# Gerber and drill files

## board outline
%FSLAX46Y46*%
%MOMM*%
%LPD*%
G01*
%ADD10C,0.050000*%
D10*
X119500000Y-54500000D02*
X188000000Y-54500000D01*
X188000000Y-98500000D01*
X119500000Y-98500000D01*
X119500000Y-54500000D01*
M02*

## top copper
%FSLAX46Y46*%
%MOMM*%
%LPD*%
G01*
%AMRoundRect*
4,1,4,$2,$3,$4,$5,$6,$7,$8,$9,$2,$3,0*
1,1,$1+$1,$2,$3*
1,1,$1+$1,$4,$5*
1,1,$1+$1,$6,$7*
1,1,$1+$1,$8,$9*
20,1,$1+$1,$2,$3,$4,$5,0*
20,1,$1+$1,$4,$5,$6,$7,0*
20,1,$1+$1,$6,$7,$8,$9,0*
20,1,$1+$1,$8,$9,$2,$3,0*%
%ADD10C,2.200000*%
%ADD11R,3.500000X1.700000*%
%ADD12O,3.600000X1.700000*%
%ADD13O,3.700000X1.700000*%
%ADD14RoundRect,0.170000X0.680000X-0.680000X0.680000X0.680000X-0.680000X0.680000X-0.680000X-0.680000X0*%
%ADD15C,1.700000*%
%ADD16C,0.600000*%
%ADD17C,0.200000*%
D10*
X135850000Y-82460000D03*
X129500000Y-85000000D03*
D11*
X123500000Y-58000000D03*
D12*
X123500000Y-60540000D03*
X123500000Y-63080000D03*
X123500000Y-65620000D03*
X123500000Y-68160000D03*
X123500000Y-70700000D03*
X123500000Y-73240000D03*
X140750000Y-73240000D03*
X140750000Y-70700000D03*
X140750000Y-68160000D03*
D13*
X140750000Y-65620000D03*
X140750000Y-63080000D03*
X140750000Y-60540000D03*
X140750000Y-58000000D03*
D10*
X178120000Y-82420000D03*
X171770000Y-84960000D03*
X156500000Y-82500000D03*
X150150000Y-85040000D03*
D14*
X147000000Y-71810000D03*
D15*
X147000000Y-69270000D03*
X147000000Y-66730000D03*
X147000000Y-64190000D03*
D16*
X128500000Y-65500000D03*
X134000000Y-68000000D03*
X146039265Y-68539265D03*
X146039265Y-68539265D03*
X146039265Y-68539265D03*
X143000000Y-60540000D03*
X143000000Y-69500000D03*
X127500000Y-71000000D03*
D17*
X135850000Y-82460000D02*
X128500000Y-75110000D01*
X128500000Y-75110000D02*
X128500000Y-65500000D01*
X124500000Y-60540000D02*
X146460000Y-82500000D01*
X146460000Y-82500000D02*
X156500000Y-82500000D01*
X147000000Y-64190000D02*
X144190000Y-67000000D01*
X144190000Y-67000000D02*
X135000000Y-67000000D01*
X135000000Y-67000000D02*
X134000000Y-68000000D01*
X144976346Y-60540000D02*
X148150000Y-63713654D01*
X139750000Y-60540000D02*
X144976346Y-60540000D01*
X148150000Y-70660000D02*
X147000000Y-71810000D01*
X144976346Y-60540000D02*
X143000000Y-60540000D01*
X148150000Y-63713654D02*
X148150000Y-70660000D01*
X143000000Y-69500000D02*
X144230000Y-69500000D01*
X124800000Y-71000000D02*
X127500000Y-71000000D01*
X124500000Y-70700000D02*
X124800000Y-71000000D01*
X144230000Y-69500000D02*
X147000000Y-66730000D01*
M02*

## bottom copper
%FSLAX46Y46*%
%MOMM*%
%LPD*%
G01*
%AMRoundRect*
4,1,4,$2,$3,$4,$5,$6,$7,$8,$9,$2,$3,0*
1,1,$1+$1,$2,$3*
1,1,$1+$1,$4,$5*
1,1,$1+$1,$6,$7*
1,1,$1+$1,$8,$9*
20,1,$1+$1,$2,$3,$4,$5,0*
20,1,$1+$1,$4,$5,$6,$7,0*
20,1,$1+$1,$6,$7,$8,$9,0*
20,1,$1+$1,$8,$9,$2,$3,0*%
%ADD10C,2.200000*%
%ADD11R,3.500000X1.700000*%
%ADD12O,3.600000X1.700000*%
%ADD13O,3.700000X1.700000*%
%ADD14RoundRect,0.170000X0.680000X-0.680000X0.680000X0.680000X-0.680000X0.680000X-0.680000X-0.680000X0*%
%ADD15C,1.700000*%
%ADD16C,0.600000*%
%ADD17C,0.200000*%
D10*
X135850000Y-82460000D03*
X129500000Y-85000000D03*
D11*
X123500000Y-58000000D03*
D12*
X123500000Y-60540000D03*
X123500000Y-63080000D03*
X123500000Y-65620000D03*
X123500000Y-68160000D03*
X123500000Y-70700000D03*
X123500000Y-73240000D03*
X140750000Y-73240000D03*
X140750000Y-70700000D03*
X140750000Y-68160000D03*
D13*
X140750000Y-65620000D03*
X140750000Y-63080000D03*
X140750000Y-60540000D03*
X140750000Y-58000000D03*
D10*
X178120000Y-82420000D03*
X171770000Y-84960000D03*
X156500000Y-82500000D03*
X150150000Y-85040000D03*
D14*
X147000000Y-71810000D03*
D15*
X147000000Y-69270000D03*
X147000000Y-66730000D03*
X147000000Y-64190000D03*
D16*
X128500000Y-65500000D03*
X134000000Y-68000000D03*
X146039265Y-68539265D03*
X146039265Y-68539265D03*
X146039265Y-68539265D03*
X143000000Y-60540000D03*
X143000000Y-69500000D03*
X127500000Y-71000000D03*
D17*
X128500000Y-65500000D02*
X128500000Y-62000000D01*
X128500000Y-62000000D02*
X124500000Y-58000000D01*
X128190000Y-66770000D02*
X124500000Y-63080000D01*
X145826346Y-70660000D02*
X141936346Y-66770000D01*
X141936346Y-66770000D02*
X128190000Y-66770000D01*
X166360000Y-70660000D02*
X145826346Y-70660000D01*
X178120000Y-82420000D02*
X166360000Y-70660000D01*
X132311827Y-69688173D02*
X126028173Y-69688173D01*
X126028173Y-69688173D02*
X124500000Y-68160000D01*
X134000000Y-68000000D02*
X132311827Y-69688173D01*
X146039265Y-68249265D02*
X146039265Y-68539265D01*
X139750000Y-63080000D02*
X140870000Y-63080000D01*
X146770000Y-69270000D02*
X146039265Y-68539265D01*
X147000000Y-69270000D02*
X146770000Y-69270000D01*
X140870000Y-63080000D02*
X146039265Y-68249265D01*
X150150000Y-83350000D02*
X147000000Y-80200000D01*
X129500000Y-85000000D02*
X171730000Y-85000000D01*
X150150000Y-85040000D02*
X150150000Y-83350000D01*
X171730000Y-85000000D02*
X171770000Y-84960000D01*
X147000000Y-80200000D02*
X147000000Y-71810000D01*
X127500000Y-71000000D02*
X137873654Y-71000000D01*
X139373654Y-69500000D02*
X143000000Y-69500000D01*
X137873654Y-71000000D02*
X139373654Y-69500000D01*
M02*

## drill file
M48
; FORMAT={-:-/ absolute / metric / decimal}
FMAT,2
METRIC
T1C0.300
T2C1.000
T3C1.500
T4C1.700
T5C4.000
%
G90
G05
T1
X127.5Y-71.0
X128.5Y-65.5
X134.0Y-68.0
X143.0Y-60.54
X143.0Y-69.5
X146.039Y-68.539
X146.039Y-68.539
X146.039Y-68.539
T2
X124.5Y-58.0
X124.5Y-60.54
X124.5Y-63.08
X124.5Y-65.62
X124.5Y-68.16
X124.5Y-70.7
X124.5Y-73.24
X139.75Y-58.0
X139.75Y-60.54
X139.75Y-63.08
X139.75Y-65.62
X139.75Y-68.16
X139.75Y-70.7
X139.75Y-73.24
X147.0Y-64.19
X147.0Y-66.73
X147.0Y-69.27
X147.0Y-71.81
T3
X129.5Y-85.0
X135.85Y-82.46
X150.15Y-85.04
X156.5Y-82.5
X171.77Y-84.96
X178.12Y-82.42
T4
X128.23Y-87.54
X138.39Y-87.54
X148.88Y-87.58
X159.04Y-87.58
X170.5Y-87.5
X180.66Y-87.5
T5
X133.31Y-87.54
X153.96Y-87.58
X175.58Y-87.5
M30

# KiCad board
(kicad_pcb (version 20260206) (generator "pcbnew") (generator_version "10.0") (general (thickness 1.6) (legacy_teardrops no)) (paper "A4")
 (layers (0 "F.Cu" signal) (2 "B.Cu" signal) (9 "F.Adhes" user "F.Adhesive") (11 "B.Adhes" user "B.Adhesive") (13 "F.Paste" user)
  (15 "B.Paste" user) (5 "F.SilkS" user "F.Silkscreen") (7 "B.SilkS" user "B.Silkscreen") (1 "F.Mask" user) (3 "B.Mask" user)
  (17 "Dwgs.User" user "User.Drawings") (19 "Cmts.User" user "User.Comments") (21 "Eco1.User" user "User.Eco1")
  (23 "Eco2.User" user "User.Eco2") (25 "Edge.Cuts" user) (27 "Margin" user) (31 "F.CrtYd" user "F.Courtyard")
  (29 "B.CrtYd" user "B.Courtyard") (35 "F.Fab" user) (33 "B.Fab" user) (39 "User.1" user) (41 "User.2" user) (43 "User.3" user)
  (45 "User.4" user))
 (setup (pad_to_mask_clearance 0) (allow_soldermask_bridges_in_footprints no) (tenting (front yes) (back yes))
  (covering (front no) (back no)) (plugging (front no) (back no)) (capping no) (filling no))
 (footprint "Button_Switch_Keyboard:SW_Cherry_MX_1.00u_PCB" (layer "F.Cu") (at 135.85 82.46)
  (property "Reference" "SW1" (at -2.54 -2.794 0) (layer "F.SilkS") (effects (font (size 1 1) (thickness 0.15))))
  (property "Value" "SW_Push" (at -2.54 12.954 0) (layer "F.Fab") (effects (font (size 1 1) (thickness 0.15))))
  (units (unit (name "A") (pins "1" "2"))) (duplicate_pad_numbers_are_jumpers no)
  (pad "" np_thru_hole circle (at -7.62 5.08) (size 1.7 1.7) (drill 1.7) (layers "*.Cu" "*.Mask"))
  (pad "" np_thru_hole circle (at -2.54 5.08) (size 4 4) (drill 4) (layers "*.Cu" "*.Mask"))
  (pad "" np_thru_hole circle (at 2.54 5.08) (size 1.7 1.7) (drill 1.7) (layers "*.Cu" "*.Mask"))
  (pad "1" thru_hole circle (at 0 0) (size 2.2 2.2) (drill 1.5) (layers "*.Cu" "*.Mask") (remove_unused_layers no)
   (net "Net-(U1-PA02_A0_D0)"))
  (pad "2" thru_hole circle (at -6.35 2.54) (size 2.2 2.2) (drill 1.5) (layers "*.Cu" "*.Mask") (remove_unused_layers no)
   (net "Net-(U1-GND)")))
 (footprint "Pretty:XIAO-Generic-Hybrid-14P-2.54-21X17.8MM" (layer "F.Cu") (at 132.125 65.62)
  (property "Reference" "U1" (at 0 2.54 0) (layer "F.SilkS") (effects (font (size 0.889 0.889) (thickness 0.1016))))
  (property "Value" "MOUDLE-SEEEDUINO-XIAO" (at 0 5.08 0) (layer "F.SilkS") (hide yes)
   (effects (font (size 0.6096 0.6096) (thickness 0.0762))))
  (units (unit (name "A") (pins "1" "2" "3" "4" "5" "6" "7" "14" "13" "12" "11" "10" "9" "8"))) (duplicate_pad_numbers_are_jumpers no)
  (pad "1" thru_hole rect (at -7.625 -7.62) (size 3.5 1.7) (drill 1 (offset -1 0)) (layers "*.Cu" "*.Mask") (remove_unused_layers no)
   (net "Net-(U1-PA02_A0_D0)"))
  (pad "2" thru_hole oval (at -7.625 -5.08) (size 3.6 1.7) (drill 1 (offset -1 0)) (layers "*.Cu" "*.Mask") (remove_unused_layers no)
   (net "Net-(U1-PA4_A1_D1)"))
  (pad "3" thru_hole oval (at -7.625 -2.54) (size 3.6 1.7) (drill 1 (offset -1 0)) (layers "*.Cu" "*.Mask") (remove_unused_layers no)
   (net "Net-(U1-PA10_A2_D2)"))
  (pad "4" thru_hole oval (at -7.625 0) (size 3.6 1.7) (drill 1 (offset -1 0)) (layers "*.Cu" "*.Mask") (remove_unused_layers no)
   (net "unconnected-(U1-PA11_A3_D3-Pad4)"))
  (pad "5" thru_hole oval (at -7.625 2.54) (size 3.6 1.7) (drill 1 (offset -1 0)) (layers "*.Cu" "*.Mask") (remove_unused_layers no)
   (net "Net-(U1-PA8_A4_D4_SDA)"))
  (pad "6" thru_hole oval (at -7.625 5.08 180) (size 3.6 1.7) (drill 1 (offset 1 0)) (layers "*.Cu" "*.Mask") (remove_unused_layers no)
   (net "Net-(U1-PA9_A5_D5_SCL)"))
  (pad "7" thru_hole oval (at -7.625 7.62) (size 3.6 1.7) (drill 1 (offset -1 0)) (layers "*.Cu" "*.Mask") (remove_unused_layers no)
   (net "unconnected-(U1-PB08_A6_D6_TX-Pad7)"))
  (pad "8" thru_hole oval (at 7.625 7.62) (size 3.6 1.7) (drill 1 (offset 1 0)) (layers "*.Cu" "*.Mask") (remove_unused_layers no)
   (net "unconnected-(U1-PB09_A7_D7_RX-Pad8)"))
  (pad "9" thru_hole oval (at 7.625 5.08) (size 3.6 1.7) (drill 1 (offset 1 0)) (layers "*.Cu" "*.Mask") (remove_unused_layers no)
   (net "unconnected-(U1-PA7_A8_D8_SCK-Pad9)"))
  (pad "10" thru_hole oval (at 7.625 2.54) (size 3.6 1.7) (drill 1 (offset 1 0)) (layers "*.Cu" "*.Mask") (remove_unused_layers no)
   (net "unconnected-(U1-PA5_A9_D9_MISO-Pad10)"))
  (pad "11" thru_hole oval (at 7.625 0) (size 3.7 1.7) (drill 1 (offset 1 0)) (layers "*.Cu" "*.Mask") (remove_unused_layers no)
   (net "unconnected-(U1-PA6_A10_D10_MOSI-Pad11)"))
  (pad "12" thru_hole oval (at 7.625 -2.54) (size 3.7 1.7) (drill 1 (offset 1 0)) (layers "*.Cu" "*.Mask") (remove_unused_layers no)
   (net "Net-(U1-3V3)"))
  (pad "13" thru_hole oval (at 7.625 -5.08) (size 3.7 1.7) (drill 1 (offset 1 0)) (layers "*.Cu" "*.Mask") (remove_unused_layers no)
   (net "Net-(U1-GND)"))
  (pad "14" thru_hole oval (at 7.625 -7.62) (size 3.7 1.7) (drill 1 (offset 1 0)) (layers "*.Cu" "*.Mask") (remove_unused_layers no)
   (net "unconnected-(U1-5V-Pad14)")))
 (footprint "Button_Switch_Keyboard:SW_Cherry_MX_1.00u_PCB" (layer "F.Cu") (at 178.12 82.42)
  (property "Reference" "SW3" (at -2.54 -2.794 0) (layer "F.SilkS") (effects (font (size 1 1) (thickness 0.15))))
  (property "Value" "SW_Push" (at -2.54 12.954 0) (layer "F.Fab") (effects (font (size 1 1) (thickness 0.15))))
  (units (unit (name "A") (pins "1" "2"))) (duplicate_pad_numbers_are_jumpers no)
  (pad "" np_thru_hole circle (at -7.62 5.08) (size 1.7 1.7) (drill 1.7) (layers "*.Cu" "*.Mask"))
  (pad "" np_thru_hole circle (at -2.54 5.08) (size 4 4) (drill 4) (layers "*.Cu" "*.Mask"))
  (pad "" np_thru_hole circle (at 2.54 5.08) (size 1.7 1.7) (drill 1.7) (layers "*.Cu" "*.Mask"))
  (pad "1" thru_hole circle (at 0 0) (size 2.2 2.2) (drill 1.5) (layers "*.Cu" "*.Mask") (remove_unused_layers no)
   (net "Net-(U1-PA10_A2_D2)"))
  (pad "2" thru_hole circle (at -6.35 2.54) (size 2.2 2.2) (drill 1.5) (layers "*.Cu" "*.Mask") (remove_unused_layers no)
   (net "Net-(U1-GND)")))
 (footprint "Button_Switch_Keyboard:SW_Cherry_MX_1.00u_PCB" (layer "F.Cu") (at 156.5 82.5)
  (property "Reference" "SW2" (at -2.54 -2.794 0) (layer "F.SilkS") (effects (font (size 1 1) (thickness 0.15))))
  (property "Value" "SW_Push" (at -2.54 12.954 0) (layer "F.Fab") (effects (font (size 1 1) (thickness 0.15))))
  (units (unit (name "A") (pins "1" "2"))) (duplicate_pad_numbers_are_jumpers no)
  (pad "" np_thru_hole circle (at -7.62 5.08) (size 1.7 1.7) (drill 1.7) (layers "*.Cu" "*.Mask"))
  (pad "" np_thru_hole circle (at -2.54 5.08) (size 4 4) (drill 4) (layers "*.Cu" "*.Mask"))
  (pad "" np_thru_hole circle (at 2.54 5.08) (size 1.7 1.7) (drill 1.7) (layers "*.Cu" "*.Mask"))
  (pad "1" thru_hole circle (at 0 0) (size 2.2 2.2) (drill 1.5) (layers "*.Cu" "*.Mask") (remove_unused_layers no)
   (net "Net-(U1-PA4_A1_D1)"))
  (pad "2" thru_hole circle (at -6.35 2.54) (size 2.2 2.2) (drill 1.5) (layers "*.Cu" "*.Mask") (remove_unused_layers no)
   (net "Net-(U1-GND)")))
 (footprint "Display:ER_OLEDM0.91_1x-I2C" (layer "F.Cu") (at 147 71.81 90)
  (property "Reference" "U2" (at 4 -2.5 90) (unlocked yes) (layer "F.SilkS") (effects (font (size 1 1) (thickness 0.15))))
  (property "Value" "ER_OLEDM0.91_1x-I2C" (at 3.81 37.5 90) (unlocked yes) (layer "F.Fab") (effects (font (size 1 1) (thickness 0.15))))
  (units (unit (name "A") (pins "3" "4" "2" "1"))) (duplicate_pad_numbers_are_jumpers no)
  (pad "1" thru_hole roundrect (at 0 0 90) (size 1.7 1.7) (drill 1) (layers "*.Cu" "*.Mask") (remove_unused_layers no)
   (roundrect_rratio 0.1) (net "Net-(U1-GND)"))
  (pad "2" thru_hole circle (at 2.54 0 90) (size 1.7 1.7) (drill 1) (layers "*.Cu" "*.Mask") (remove_unused_layers no) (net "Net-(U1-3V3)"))
  (pad "3" thru_hole circle (at 5.08 0 90) (size 1.7 1.7) (drill 1) (layers "*.Cu" "*.Mask") (remove_unused_layers no)
   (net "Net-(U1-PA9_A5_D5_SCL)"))
  (pad "4" thru_hole circle (at 7.62 0 90) (size 1.7 1.7) (drill 1) (layers "*.Cu" "*.Mask") (remove_unused_layers no)
   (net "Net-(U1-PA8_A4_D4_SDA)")))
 (gr_rect (start 119.5 54.5) (end 188 98.5) (stroke (width 0.05) (type default)) (fill no) (layer "Edge.Cuts"))
 (segment (start 135.85 82.46) (end 128.5 75.11) (width 0.2) (layer "F.Cu") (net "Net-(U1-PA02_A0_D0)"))
 (segment (start 128.5 75.11) (end 128.5 65.5) (width 0.2) (layer "F.Cu") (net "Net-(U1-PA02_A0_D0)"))
 (via (at 128.5 65.5) (size 0.6) (drill 0.3) (layers "F.Cu" "B.Cu") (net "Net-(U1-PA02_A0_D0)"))
 (segment (start 128.5 65.5) (end 128.5 62) (width 0.2) (layer "B.Cu") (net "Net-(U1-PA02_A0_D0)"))
 (segment (start 128.5 62) (end 124.5 58) (width 0.2) (layer "B.Cu") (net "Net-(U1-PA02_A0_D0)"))
 (segment (start 124.5 60.54) (end 146.46 82.5) (width 0.2) (layer "F.Cu") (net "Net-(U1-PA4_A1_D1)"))
 (segment (start 146.46 82.5) (end 156.5 82.5) (width 0.2) (layer "F.Cu") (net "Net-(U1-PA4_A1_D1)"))
 (segment (start 128.19 66.77) (end 124.5 63.08) (width 0.2) (layer "B.Cu") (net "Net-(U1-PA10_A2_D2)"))
 (segment (start 145.826346 70.66) (end 141.936346 66.77) (width 0.2) (layer "B.Cu") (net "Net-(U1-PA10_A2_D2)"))
 (segment (start 141.936346 66.77) (end 128.19 66.77) (width 0.2) (layer "B.Cu") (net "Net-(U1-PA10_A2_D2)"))
 (segment (start 166.36 70.66) (end 145.826346 70.66) (width 0.2) (layer "B.Cu") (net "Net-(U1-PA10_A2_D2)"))
 (segment (start 178.12 82.42) (end 166.36 70.66) (width 0.2) (layer "B.Cu") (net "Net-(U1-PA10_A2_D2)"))
 (segment (start 147 64.19) (end 144.19 67) (width 0.2) (layer "F.Cu") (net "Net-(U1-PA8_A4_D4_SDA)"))
 (segment (start 144.19 67) (end 135 67) (width 0.2) (layer "F.Cu") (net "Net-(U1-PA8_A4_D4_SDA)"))
 (segment (start 135 67) (end 134 68) (width 0.2) (layer "F.Cu") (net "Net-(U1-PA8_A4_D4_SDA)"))
 (via (at 134 68) (size 0.6) (drill 0.3) (layers "F.Cu" "B.Cu") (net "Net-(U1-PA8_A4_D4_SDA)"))
 (segment (start 132.311827 69.688173) (end 126.028173 69.688173) (width 0.2) (layer "B.Cu") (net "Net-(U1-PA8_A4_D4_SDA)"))
 (segment (start 126.028173 69.688173) (end 124.5 68.16) (width 0.2) (layer "B.Cu") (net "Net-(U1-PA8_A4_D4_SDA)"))
 (segment (start 134 68) (end 132.311827 69.688173) (width 0.2) (layer "B.Cu") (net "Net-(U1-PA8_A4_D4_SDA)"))
 (via (at 146.039265 68.539265) (size 0.6) (drill 0.3) (layers "F.Cu" "B.Cu") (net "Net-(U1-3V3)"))
 (via (at 146.039265 68.539265) (size 0.6) (drill 0.3) (layers "F.Cu" "B.Cu") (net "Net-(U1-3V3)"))
 (via (at 146.039265 68.539265) (size 0.6) (drill 0.3) (layers "F.Cu" "B.Cu") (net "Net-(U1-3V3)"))
 (segment (start 146.039265 68.249265) (end 146.039265 68.539265) (width 0.2) (layer "B.Cu") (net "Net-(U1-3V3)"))
 (segment (start 139.75 63.08) (end 140.87 63.08) (width 0.2) (layer "B.Cu") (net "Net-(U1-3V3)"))
 (segment (start 146.77 69.27) (end 146.039265 68.539265) (width 0.2) (layer "B.Cu") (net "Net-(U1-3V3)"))
 (segment (start 147 69.27) (end 146.77 69.27) (width 0.2) (layer "B.Cu") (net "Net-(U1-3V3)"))
 (segment (start 140.87 63.08) (end 146.039265 68.249265) (width 0.2) (layer "B.Cu") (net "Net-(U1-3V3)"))
 (segment (start 144.976346 60.54) (end 148.15 63.713654) (width 0.2) (layer "F.Cu") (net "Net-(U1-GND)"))
 (segment (start 139.75 60.54) (end 144.976346 60.54) (width 0.2) (layer "F.Cu") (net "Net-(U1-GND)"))
 (segment (start 148.15 70.66) (end 147 71.81) (width 0.2) (layer "F.Cu") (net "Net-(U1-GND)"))
 (segment (start 144.976346 60.54) (end 143 60.54) (width 0.2) (layer "F.Cu") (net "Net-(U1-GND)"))
 (segment (start 148.15 63.713654) (end 148.15 70.66) (width 0.2) (layer "F.Cu") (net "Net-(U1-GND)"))
 (via (at 143 60.54) (size 0.6) (drill 0.3) (layers "F.Cu" "B.Cu") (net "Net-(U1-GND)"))
 (segment (start 150.15 83.35) (end 147 80.2) (width 0.2) (layer "B.Cu") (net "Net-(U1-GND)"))
 (segment (start 129.5 85) (end 171.73 85) (width 0.2) (layer "B.Cu") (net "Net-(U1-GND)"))
 (segment (start 150.15 85.04) (end 150.15 83.35) (width 0.2) (layer "B.Cu") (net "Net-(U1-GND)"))
 (segment (start 171.73 85) (end 171.77 84.96) (width 0.2) (layer "B.Cu") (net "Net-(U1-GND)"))
 (segment (start 147 80.2) (end 147 71.81) (width 0.2) (layer "B.Cu") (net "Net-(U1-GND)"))
 (segment (start 143 69.5) (end 144.23 69.5) (width 0.2) (layer "F.Cu") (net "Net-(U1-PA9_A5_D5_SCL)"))
 (segment (start 124.8 71) (end 127.5 71) (width 0.2) (layer "F.Cu") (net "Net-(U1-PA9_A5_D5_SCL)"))
 (segment (start 124.5 70.7) (end 124.8 71) (width 0.2) (layer "F.Cu") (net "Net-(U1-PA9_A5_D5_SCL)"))
 (segment (start 144.23 69.5) (end 147 66.73) (width 0.2) (layer "F.Cu") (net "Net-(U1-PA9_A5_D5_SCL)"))
 (via (at 143 69.5) (size 0.6) (drill 0.3) (layers "F.Cu" "B.Cu") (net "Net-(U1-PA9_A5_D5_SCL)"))
 (via (at 127.5 71) (size 0.6) (drill 0.3) (layers "F.Cu" "B.Cu") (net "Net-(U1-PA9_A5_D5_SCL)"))
 (segment (start 127.5 71) (end 137.873654 71) (width 0.2) (layer "B.Cu") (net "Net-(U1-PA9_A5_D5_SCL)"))
 (segment (start 139.373654 69.5) (end 143 69.5) (width 0.2) (layer "B.Cu") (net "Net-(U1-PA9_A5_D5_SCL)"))
 (segment (start 137.873654 71) (end 139.373654 69.5) (width 0.2) (layer "B.Cu") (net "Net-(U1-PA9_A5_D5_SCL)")))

